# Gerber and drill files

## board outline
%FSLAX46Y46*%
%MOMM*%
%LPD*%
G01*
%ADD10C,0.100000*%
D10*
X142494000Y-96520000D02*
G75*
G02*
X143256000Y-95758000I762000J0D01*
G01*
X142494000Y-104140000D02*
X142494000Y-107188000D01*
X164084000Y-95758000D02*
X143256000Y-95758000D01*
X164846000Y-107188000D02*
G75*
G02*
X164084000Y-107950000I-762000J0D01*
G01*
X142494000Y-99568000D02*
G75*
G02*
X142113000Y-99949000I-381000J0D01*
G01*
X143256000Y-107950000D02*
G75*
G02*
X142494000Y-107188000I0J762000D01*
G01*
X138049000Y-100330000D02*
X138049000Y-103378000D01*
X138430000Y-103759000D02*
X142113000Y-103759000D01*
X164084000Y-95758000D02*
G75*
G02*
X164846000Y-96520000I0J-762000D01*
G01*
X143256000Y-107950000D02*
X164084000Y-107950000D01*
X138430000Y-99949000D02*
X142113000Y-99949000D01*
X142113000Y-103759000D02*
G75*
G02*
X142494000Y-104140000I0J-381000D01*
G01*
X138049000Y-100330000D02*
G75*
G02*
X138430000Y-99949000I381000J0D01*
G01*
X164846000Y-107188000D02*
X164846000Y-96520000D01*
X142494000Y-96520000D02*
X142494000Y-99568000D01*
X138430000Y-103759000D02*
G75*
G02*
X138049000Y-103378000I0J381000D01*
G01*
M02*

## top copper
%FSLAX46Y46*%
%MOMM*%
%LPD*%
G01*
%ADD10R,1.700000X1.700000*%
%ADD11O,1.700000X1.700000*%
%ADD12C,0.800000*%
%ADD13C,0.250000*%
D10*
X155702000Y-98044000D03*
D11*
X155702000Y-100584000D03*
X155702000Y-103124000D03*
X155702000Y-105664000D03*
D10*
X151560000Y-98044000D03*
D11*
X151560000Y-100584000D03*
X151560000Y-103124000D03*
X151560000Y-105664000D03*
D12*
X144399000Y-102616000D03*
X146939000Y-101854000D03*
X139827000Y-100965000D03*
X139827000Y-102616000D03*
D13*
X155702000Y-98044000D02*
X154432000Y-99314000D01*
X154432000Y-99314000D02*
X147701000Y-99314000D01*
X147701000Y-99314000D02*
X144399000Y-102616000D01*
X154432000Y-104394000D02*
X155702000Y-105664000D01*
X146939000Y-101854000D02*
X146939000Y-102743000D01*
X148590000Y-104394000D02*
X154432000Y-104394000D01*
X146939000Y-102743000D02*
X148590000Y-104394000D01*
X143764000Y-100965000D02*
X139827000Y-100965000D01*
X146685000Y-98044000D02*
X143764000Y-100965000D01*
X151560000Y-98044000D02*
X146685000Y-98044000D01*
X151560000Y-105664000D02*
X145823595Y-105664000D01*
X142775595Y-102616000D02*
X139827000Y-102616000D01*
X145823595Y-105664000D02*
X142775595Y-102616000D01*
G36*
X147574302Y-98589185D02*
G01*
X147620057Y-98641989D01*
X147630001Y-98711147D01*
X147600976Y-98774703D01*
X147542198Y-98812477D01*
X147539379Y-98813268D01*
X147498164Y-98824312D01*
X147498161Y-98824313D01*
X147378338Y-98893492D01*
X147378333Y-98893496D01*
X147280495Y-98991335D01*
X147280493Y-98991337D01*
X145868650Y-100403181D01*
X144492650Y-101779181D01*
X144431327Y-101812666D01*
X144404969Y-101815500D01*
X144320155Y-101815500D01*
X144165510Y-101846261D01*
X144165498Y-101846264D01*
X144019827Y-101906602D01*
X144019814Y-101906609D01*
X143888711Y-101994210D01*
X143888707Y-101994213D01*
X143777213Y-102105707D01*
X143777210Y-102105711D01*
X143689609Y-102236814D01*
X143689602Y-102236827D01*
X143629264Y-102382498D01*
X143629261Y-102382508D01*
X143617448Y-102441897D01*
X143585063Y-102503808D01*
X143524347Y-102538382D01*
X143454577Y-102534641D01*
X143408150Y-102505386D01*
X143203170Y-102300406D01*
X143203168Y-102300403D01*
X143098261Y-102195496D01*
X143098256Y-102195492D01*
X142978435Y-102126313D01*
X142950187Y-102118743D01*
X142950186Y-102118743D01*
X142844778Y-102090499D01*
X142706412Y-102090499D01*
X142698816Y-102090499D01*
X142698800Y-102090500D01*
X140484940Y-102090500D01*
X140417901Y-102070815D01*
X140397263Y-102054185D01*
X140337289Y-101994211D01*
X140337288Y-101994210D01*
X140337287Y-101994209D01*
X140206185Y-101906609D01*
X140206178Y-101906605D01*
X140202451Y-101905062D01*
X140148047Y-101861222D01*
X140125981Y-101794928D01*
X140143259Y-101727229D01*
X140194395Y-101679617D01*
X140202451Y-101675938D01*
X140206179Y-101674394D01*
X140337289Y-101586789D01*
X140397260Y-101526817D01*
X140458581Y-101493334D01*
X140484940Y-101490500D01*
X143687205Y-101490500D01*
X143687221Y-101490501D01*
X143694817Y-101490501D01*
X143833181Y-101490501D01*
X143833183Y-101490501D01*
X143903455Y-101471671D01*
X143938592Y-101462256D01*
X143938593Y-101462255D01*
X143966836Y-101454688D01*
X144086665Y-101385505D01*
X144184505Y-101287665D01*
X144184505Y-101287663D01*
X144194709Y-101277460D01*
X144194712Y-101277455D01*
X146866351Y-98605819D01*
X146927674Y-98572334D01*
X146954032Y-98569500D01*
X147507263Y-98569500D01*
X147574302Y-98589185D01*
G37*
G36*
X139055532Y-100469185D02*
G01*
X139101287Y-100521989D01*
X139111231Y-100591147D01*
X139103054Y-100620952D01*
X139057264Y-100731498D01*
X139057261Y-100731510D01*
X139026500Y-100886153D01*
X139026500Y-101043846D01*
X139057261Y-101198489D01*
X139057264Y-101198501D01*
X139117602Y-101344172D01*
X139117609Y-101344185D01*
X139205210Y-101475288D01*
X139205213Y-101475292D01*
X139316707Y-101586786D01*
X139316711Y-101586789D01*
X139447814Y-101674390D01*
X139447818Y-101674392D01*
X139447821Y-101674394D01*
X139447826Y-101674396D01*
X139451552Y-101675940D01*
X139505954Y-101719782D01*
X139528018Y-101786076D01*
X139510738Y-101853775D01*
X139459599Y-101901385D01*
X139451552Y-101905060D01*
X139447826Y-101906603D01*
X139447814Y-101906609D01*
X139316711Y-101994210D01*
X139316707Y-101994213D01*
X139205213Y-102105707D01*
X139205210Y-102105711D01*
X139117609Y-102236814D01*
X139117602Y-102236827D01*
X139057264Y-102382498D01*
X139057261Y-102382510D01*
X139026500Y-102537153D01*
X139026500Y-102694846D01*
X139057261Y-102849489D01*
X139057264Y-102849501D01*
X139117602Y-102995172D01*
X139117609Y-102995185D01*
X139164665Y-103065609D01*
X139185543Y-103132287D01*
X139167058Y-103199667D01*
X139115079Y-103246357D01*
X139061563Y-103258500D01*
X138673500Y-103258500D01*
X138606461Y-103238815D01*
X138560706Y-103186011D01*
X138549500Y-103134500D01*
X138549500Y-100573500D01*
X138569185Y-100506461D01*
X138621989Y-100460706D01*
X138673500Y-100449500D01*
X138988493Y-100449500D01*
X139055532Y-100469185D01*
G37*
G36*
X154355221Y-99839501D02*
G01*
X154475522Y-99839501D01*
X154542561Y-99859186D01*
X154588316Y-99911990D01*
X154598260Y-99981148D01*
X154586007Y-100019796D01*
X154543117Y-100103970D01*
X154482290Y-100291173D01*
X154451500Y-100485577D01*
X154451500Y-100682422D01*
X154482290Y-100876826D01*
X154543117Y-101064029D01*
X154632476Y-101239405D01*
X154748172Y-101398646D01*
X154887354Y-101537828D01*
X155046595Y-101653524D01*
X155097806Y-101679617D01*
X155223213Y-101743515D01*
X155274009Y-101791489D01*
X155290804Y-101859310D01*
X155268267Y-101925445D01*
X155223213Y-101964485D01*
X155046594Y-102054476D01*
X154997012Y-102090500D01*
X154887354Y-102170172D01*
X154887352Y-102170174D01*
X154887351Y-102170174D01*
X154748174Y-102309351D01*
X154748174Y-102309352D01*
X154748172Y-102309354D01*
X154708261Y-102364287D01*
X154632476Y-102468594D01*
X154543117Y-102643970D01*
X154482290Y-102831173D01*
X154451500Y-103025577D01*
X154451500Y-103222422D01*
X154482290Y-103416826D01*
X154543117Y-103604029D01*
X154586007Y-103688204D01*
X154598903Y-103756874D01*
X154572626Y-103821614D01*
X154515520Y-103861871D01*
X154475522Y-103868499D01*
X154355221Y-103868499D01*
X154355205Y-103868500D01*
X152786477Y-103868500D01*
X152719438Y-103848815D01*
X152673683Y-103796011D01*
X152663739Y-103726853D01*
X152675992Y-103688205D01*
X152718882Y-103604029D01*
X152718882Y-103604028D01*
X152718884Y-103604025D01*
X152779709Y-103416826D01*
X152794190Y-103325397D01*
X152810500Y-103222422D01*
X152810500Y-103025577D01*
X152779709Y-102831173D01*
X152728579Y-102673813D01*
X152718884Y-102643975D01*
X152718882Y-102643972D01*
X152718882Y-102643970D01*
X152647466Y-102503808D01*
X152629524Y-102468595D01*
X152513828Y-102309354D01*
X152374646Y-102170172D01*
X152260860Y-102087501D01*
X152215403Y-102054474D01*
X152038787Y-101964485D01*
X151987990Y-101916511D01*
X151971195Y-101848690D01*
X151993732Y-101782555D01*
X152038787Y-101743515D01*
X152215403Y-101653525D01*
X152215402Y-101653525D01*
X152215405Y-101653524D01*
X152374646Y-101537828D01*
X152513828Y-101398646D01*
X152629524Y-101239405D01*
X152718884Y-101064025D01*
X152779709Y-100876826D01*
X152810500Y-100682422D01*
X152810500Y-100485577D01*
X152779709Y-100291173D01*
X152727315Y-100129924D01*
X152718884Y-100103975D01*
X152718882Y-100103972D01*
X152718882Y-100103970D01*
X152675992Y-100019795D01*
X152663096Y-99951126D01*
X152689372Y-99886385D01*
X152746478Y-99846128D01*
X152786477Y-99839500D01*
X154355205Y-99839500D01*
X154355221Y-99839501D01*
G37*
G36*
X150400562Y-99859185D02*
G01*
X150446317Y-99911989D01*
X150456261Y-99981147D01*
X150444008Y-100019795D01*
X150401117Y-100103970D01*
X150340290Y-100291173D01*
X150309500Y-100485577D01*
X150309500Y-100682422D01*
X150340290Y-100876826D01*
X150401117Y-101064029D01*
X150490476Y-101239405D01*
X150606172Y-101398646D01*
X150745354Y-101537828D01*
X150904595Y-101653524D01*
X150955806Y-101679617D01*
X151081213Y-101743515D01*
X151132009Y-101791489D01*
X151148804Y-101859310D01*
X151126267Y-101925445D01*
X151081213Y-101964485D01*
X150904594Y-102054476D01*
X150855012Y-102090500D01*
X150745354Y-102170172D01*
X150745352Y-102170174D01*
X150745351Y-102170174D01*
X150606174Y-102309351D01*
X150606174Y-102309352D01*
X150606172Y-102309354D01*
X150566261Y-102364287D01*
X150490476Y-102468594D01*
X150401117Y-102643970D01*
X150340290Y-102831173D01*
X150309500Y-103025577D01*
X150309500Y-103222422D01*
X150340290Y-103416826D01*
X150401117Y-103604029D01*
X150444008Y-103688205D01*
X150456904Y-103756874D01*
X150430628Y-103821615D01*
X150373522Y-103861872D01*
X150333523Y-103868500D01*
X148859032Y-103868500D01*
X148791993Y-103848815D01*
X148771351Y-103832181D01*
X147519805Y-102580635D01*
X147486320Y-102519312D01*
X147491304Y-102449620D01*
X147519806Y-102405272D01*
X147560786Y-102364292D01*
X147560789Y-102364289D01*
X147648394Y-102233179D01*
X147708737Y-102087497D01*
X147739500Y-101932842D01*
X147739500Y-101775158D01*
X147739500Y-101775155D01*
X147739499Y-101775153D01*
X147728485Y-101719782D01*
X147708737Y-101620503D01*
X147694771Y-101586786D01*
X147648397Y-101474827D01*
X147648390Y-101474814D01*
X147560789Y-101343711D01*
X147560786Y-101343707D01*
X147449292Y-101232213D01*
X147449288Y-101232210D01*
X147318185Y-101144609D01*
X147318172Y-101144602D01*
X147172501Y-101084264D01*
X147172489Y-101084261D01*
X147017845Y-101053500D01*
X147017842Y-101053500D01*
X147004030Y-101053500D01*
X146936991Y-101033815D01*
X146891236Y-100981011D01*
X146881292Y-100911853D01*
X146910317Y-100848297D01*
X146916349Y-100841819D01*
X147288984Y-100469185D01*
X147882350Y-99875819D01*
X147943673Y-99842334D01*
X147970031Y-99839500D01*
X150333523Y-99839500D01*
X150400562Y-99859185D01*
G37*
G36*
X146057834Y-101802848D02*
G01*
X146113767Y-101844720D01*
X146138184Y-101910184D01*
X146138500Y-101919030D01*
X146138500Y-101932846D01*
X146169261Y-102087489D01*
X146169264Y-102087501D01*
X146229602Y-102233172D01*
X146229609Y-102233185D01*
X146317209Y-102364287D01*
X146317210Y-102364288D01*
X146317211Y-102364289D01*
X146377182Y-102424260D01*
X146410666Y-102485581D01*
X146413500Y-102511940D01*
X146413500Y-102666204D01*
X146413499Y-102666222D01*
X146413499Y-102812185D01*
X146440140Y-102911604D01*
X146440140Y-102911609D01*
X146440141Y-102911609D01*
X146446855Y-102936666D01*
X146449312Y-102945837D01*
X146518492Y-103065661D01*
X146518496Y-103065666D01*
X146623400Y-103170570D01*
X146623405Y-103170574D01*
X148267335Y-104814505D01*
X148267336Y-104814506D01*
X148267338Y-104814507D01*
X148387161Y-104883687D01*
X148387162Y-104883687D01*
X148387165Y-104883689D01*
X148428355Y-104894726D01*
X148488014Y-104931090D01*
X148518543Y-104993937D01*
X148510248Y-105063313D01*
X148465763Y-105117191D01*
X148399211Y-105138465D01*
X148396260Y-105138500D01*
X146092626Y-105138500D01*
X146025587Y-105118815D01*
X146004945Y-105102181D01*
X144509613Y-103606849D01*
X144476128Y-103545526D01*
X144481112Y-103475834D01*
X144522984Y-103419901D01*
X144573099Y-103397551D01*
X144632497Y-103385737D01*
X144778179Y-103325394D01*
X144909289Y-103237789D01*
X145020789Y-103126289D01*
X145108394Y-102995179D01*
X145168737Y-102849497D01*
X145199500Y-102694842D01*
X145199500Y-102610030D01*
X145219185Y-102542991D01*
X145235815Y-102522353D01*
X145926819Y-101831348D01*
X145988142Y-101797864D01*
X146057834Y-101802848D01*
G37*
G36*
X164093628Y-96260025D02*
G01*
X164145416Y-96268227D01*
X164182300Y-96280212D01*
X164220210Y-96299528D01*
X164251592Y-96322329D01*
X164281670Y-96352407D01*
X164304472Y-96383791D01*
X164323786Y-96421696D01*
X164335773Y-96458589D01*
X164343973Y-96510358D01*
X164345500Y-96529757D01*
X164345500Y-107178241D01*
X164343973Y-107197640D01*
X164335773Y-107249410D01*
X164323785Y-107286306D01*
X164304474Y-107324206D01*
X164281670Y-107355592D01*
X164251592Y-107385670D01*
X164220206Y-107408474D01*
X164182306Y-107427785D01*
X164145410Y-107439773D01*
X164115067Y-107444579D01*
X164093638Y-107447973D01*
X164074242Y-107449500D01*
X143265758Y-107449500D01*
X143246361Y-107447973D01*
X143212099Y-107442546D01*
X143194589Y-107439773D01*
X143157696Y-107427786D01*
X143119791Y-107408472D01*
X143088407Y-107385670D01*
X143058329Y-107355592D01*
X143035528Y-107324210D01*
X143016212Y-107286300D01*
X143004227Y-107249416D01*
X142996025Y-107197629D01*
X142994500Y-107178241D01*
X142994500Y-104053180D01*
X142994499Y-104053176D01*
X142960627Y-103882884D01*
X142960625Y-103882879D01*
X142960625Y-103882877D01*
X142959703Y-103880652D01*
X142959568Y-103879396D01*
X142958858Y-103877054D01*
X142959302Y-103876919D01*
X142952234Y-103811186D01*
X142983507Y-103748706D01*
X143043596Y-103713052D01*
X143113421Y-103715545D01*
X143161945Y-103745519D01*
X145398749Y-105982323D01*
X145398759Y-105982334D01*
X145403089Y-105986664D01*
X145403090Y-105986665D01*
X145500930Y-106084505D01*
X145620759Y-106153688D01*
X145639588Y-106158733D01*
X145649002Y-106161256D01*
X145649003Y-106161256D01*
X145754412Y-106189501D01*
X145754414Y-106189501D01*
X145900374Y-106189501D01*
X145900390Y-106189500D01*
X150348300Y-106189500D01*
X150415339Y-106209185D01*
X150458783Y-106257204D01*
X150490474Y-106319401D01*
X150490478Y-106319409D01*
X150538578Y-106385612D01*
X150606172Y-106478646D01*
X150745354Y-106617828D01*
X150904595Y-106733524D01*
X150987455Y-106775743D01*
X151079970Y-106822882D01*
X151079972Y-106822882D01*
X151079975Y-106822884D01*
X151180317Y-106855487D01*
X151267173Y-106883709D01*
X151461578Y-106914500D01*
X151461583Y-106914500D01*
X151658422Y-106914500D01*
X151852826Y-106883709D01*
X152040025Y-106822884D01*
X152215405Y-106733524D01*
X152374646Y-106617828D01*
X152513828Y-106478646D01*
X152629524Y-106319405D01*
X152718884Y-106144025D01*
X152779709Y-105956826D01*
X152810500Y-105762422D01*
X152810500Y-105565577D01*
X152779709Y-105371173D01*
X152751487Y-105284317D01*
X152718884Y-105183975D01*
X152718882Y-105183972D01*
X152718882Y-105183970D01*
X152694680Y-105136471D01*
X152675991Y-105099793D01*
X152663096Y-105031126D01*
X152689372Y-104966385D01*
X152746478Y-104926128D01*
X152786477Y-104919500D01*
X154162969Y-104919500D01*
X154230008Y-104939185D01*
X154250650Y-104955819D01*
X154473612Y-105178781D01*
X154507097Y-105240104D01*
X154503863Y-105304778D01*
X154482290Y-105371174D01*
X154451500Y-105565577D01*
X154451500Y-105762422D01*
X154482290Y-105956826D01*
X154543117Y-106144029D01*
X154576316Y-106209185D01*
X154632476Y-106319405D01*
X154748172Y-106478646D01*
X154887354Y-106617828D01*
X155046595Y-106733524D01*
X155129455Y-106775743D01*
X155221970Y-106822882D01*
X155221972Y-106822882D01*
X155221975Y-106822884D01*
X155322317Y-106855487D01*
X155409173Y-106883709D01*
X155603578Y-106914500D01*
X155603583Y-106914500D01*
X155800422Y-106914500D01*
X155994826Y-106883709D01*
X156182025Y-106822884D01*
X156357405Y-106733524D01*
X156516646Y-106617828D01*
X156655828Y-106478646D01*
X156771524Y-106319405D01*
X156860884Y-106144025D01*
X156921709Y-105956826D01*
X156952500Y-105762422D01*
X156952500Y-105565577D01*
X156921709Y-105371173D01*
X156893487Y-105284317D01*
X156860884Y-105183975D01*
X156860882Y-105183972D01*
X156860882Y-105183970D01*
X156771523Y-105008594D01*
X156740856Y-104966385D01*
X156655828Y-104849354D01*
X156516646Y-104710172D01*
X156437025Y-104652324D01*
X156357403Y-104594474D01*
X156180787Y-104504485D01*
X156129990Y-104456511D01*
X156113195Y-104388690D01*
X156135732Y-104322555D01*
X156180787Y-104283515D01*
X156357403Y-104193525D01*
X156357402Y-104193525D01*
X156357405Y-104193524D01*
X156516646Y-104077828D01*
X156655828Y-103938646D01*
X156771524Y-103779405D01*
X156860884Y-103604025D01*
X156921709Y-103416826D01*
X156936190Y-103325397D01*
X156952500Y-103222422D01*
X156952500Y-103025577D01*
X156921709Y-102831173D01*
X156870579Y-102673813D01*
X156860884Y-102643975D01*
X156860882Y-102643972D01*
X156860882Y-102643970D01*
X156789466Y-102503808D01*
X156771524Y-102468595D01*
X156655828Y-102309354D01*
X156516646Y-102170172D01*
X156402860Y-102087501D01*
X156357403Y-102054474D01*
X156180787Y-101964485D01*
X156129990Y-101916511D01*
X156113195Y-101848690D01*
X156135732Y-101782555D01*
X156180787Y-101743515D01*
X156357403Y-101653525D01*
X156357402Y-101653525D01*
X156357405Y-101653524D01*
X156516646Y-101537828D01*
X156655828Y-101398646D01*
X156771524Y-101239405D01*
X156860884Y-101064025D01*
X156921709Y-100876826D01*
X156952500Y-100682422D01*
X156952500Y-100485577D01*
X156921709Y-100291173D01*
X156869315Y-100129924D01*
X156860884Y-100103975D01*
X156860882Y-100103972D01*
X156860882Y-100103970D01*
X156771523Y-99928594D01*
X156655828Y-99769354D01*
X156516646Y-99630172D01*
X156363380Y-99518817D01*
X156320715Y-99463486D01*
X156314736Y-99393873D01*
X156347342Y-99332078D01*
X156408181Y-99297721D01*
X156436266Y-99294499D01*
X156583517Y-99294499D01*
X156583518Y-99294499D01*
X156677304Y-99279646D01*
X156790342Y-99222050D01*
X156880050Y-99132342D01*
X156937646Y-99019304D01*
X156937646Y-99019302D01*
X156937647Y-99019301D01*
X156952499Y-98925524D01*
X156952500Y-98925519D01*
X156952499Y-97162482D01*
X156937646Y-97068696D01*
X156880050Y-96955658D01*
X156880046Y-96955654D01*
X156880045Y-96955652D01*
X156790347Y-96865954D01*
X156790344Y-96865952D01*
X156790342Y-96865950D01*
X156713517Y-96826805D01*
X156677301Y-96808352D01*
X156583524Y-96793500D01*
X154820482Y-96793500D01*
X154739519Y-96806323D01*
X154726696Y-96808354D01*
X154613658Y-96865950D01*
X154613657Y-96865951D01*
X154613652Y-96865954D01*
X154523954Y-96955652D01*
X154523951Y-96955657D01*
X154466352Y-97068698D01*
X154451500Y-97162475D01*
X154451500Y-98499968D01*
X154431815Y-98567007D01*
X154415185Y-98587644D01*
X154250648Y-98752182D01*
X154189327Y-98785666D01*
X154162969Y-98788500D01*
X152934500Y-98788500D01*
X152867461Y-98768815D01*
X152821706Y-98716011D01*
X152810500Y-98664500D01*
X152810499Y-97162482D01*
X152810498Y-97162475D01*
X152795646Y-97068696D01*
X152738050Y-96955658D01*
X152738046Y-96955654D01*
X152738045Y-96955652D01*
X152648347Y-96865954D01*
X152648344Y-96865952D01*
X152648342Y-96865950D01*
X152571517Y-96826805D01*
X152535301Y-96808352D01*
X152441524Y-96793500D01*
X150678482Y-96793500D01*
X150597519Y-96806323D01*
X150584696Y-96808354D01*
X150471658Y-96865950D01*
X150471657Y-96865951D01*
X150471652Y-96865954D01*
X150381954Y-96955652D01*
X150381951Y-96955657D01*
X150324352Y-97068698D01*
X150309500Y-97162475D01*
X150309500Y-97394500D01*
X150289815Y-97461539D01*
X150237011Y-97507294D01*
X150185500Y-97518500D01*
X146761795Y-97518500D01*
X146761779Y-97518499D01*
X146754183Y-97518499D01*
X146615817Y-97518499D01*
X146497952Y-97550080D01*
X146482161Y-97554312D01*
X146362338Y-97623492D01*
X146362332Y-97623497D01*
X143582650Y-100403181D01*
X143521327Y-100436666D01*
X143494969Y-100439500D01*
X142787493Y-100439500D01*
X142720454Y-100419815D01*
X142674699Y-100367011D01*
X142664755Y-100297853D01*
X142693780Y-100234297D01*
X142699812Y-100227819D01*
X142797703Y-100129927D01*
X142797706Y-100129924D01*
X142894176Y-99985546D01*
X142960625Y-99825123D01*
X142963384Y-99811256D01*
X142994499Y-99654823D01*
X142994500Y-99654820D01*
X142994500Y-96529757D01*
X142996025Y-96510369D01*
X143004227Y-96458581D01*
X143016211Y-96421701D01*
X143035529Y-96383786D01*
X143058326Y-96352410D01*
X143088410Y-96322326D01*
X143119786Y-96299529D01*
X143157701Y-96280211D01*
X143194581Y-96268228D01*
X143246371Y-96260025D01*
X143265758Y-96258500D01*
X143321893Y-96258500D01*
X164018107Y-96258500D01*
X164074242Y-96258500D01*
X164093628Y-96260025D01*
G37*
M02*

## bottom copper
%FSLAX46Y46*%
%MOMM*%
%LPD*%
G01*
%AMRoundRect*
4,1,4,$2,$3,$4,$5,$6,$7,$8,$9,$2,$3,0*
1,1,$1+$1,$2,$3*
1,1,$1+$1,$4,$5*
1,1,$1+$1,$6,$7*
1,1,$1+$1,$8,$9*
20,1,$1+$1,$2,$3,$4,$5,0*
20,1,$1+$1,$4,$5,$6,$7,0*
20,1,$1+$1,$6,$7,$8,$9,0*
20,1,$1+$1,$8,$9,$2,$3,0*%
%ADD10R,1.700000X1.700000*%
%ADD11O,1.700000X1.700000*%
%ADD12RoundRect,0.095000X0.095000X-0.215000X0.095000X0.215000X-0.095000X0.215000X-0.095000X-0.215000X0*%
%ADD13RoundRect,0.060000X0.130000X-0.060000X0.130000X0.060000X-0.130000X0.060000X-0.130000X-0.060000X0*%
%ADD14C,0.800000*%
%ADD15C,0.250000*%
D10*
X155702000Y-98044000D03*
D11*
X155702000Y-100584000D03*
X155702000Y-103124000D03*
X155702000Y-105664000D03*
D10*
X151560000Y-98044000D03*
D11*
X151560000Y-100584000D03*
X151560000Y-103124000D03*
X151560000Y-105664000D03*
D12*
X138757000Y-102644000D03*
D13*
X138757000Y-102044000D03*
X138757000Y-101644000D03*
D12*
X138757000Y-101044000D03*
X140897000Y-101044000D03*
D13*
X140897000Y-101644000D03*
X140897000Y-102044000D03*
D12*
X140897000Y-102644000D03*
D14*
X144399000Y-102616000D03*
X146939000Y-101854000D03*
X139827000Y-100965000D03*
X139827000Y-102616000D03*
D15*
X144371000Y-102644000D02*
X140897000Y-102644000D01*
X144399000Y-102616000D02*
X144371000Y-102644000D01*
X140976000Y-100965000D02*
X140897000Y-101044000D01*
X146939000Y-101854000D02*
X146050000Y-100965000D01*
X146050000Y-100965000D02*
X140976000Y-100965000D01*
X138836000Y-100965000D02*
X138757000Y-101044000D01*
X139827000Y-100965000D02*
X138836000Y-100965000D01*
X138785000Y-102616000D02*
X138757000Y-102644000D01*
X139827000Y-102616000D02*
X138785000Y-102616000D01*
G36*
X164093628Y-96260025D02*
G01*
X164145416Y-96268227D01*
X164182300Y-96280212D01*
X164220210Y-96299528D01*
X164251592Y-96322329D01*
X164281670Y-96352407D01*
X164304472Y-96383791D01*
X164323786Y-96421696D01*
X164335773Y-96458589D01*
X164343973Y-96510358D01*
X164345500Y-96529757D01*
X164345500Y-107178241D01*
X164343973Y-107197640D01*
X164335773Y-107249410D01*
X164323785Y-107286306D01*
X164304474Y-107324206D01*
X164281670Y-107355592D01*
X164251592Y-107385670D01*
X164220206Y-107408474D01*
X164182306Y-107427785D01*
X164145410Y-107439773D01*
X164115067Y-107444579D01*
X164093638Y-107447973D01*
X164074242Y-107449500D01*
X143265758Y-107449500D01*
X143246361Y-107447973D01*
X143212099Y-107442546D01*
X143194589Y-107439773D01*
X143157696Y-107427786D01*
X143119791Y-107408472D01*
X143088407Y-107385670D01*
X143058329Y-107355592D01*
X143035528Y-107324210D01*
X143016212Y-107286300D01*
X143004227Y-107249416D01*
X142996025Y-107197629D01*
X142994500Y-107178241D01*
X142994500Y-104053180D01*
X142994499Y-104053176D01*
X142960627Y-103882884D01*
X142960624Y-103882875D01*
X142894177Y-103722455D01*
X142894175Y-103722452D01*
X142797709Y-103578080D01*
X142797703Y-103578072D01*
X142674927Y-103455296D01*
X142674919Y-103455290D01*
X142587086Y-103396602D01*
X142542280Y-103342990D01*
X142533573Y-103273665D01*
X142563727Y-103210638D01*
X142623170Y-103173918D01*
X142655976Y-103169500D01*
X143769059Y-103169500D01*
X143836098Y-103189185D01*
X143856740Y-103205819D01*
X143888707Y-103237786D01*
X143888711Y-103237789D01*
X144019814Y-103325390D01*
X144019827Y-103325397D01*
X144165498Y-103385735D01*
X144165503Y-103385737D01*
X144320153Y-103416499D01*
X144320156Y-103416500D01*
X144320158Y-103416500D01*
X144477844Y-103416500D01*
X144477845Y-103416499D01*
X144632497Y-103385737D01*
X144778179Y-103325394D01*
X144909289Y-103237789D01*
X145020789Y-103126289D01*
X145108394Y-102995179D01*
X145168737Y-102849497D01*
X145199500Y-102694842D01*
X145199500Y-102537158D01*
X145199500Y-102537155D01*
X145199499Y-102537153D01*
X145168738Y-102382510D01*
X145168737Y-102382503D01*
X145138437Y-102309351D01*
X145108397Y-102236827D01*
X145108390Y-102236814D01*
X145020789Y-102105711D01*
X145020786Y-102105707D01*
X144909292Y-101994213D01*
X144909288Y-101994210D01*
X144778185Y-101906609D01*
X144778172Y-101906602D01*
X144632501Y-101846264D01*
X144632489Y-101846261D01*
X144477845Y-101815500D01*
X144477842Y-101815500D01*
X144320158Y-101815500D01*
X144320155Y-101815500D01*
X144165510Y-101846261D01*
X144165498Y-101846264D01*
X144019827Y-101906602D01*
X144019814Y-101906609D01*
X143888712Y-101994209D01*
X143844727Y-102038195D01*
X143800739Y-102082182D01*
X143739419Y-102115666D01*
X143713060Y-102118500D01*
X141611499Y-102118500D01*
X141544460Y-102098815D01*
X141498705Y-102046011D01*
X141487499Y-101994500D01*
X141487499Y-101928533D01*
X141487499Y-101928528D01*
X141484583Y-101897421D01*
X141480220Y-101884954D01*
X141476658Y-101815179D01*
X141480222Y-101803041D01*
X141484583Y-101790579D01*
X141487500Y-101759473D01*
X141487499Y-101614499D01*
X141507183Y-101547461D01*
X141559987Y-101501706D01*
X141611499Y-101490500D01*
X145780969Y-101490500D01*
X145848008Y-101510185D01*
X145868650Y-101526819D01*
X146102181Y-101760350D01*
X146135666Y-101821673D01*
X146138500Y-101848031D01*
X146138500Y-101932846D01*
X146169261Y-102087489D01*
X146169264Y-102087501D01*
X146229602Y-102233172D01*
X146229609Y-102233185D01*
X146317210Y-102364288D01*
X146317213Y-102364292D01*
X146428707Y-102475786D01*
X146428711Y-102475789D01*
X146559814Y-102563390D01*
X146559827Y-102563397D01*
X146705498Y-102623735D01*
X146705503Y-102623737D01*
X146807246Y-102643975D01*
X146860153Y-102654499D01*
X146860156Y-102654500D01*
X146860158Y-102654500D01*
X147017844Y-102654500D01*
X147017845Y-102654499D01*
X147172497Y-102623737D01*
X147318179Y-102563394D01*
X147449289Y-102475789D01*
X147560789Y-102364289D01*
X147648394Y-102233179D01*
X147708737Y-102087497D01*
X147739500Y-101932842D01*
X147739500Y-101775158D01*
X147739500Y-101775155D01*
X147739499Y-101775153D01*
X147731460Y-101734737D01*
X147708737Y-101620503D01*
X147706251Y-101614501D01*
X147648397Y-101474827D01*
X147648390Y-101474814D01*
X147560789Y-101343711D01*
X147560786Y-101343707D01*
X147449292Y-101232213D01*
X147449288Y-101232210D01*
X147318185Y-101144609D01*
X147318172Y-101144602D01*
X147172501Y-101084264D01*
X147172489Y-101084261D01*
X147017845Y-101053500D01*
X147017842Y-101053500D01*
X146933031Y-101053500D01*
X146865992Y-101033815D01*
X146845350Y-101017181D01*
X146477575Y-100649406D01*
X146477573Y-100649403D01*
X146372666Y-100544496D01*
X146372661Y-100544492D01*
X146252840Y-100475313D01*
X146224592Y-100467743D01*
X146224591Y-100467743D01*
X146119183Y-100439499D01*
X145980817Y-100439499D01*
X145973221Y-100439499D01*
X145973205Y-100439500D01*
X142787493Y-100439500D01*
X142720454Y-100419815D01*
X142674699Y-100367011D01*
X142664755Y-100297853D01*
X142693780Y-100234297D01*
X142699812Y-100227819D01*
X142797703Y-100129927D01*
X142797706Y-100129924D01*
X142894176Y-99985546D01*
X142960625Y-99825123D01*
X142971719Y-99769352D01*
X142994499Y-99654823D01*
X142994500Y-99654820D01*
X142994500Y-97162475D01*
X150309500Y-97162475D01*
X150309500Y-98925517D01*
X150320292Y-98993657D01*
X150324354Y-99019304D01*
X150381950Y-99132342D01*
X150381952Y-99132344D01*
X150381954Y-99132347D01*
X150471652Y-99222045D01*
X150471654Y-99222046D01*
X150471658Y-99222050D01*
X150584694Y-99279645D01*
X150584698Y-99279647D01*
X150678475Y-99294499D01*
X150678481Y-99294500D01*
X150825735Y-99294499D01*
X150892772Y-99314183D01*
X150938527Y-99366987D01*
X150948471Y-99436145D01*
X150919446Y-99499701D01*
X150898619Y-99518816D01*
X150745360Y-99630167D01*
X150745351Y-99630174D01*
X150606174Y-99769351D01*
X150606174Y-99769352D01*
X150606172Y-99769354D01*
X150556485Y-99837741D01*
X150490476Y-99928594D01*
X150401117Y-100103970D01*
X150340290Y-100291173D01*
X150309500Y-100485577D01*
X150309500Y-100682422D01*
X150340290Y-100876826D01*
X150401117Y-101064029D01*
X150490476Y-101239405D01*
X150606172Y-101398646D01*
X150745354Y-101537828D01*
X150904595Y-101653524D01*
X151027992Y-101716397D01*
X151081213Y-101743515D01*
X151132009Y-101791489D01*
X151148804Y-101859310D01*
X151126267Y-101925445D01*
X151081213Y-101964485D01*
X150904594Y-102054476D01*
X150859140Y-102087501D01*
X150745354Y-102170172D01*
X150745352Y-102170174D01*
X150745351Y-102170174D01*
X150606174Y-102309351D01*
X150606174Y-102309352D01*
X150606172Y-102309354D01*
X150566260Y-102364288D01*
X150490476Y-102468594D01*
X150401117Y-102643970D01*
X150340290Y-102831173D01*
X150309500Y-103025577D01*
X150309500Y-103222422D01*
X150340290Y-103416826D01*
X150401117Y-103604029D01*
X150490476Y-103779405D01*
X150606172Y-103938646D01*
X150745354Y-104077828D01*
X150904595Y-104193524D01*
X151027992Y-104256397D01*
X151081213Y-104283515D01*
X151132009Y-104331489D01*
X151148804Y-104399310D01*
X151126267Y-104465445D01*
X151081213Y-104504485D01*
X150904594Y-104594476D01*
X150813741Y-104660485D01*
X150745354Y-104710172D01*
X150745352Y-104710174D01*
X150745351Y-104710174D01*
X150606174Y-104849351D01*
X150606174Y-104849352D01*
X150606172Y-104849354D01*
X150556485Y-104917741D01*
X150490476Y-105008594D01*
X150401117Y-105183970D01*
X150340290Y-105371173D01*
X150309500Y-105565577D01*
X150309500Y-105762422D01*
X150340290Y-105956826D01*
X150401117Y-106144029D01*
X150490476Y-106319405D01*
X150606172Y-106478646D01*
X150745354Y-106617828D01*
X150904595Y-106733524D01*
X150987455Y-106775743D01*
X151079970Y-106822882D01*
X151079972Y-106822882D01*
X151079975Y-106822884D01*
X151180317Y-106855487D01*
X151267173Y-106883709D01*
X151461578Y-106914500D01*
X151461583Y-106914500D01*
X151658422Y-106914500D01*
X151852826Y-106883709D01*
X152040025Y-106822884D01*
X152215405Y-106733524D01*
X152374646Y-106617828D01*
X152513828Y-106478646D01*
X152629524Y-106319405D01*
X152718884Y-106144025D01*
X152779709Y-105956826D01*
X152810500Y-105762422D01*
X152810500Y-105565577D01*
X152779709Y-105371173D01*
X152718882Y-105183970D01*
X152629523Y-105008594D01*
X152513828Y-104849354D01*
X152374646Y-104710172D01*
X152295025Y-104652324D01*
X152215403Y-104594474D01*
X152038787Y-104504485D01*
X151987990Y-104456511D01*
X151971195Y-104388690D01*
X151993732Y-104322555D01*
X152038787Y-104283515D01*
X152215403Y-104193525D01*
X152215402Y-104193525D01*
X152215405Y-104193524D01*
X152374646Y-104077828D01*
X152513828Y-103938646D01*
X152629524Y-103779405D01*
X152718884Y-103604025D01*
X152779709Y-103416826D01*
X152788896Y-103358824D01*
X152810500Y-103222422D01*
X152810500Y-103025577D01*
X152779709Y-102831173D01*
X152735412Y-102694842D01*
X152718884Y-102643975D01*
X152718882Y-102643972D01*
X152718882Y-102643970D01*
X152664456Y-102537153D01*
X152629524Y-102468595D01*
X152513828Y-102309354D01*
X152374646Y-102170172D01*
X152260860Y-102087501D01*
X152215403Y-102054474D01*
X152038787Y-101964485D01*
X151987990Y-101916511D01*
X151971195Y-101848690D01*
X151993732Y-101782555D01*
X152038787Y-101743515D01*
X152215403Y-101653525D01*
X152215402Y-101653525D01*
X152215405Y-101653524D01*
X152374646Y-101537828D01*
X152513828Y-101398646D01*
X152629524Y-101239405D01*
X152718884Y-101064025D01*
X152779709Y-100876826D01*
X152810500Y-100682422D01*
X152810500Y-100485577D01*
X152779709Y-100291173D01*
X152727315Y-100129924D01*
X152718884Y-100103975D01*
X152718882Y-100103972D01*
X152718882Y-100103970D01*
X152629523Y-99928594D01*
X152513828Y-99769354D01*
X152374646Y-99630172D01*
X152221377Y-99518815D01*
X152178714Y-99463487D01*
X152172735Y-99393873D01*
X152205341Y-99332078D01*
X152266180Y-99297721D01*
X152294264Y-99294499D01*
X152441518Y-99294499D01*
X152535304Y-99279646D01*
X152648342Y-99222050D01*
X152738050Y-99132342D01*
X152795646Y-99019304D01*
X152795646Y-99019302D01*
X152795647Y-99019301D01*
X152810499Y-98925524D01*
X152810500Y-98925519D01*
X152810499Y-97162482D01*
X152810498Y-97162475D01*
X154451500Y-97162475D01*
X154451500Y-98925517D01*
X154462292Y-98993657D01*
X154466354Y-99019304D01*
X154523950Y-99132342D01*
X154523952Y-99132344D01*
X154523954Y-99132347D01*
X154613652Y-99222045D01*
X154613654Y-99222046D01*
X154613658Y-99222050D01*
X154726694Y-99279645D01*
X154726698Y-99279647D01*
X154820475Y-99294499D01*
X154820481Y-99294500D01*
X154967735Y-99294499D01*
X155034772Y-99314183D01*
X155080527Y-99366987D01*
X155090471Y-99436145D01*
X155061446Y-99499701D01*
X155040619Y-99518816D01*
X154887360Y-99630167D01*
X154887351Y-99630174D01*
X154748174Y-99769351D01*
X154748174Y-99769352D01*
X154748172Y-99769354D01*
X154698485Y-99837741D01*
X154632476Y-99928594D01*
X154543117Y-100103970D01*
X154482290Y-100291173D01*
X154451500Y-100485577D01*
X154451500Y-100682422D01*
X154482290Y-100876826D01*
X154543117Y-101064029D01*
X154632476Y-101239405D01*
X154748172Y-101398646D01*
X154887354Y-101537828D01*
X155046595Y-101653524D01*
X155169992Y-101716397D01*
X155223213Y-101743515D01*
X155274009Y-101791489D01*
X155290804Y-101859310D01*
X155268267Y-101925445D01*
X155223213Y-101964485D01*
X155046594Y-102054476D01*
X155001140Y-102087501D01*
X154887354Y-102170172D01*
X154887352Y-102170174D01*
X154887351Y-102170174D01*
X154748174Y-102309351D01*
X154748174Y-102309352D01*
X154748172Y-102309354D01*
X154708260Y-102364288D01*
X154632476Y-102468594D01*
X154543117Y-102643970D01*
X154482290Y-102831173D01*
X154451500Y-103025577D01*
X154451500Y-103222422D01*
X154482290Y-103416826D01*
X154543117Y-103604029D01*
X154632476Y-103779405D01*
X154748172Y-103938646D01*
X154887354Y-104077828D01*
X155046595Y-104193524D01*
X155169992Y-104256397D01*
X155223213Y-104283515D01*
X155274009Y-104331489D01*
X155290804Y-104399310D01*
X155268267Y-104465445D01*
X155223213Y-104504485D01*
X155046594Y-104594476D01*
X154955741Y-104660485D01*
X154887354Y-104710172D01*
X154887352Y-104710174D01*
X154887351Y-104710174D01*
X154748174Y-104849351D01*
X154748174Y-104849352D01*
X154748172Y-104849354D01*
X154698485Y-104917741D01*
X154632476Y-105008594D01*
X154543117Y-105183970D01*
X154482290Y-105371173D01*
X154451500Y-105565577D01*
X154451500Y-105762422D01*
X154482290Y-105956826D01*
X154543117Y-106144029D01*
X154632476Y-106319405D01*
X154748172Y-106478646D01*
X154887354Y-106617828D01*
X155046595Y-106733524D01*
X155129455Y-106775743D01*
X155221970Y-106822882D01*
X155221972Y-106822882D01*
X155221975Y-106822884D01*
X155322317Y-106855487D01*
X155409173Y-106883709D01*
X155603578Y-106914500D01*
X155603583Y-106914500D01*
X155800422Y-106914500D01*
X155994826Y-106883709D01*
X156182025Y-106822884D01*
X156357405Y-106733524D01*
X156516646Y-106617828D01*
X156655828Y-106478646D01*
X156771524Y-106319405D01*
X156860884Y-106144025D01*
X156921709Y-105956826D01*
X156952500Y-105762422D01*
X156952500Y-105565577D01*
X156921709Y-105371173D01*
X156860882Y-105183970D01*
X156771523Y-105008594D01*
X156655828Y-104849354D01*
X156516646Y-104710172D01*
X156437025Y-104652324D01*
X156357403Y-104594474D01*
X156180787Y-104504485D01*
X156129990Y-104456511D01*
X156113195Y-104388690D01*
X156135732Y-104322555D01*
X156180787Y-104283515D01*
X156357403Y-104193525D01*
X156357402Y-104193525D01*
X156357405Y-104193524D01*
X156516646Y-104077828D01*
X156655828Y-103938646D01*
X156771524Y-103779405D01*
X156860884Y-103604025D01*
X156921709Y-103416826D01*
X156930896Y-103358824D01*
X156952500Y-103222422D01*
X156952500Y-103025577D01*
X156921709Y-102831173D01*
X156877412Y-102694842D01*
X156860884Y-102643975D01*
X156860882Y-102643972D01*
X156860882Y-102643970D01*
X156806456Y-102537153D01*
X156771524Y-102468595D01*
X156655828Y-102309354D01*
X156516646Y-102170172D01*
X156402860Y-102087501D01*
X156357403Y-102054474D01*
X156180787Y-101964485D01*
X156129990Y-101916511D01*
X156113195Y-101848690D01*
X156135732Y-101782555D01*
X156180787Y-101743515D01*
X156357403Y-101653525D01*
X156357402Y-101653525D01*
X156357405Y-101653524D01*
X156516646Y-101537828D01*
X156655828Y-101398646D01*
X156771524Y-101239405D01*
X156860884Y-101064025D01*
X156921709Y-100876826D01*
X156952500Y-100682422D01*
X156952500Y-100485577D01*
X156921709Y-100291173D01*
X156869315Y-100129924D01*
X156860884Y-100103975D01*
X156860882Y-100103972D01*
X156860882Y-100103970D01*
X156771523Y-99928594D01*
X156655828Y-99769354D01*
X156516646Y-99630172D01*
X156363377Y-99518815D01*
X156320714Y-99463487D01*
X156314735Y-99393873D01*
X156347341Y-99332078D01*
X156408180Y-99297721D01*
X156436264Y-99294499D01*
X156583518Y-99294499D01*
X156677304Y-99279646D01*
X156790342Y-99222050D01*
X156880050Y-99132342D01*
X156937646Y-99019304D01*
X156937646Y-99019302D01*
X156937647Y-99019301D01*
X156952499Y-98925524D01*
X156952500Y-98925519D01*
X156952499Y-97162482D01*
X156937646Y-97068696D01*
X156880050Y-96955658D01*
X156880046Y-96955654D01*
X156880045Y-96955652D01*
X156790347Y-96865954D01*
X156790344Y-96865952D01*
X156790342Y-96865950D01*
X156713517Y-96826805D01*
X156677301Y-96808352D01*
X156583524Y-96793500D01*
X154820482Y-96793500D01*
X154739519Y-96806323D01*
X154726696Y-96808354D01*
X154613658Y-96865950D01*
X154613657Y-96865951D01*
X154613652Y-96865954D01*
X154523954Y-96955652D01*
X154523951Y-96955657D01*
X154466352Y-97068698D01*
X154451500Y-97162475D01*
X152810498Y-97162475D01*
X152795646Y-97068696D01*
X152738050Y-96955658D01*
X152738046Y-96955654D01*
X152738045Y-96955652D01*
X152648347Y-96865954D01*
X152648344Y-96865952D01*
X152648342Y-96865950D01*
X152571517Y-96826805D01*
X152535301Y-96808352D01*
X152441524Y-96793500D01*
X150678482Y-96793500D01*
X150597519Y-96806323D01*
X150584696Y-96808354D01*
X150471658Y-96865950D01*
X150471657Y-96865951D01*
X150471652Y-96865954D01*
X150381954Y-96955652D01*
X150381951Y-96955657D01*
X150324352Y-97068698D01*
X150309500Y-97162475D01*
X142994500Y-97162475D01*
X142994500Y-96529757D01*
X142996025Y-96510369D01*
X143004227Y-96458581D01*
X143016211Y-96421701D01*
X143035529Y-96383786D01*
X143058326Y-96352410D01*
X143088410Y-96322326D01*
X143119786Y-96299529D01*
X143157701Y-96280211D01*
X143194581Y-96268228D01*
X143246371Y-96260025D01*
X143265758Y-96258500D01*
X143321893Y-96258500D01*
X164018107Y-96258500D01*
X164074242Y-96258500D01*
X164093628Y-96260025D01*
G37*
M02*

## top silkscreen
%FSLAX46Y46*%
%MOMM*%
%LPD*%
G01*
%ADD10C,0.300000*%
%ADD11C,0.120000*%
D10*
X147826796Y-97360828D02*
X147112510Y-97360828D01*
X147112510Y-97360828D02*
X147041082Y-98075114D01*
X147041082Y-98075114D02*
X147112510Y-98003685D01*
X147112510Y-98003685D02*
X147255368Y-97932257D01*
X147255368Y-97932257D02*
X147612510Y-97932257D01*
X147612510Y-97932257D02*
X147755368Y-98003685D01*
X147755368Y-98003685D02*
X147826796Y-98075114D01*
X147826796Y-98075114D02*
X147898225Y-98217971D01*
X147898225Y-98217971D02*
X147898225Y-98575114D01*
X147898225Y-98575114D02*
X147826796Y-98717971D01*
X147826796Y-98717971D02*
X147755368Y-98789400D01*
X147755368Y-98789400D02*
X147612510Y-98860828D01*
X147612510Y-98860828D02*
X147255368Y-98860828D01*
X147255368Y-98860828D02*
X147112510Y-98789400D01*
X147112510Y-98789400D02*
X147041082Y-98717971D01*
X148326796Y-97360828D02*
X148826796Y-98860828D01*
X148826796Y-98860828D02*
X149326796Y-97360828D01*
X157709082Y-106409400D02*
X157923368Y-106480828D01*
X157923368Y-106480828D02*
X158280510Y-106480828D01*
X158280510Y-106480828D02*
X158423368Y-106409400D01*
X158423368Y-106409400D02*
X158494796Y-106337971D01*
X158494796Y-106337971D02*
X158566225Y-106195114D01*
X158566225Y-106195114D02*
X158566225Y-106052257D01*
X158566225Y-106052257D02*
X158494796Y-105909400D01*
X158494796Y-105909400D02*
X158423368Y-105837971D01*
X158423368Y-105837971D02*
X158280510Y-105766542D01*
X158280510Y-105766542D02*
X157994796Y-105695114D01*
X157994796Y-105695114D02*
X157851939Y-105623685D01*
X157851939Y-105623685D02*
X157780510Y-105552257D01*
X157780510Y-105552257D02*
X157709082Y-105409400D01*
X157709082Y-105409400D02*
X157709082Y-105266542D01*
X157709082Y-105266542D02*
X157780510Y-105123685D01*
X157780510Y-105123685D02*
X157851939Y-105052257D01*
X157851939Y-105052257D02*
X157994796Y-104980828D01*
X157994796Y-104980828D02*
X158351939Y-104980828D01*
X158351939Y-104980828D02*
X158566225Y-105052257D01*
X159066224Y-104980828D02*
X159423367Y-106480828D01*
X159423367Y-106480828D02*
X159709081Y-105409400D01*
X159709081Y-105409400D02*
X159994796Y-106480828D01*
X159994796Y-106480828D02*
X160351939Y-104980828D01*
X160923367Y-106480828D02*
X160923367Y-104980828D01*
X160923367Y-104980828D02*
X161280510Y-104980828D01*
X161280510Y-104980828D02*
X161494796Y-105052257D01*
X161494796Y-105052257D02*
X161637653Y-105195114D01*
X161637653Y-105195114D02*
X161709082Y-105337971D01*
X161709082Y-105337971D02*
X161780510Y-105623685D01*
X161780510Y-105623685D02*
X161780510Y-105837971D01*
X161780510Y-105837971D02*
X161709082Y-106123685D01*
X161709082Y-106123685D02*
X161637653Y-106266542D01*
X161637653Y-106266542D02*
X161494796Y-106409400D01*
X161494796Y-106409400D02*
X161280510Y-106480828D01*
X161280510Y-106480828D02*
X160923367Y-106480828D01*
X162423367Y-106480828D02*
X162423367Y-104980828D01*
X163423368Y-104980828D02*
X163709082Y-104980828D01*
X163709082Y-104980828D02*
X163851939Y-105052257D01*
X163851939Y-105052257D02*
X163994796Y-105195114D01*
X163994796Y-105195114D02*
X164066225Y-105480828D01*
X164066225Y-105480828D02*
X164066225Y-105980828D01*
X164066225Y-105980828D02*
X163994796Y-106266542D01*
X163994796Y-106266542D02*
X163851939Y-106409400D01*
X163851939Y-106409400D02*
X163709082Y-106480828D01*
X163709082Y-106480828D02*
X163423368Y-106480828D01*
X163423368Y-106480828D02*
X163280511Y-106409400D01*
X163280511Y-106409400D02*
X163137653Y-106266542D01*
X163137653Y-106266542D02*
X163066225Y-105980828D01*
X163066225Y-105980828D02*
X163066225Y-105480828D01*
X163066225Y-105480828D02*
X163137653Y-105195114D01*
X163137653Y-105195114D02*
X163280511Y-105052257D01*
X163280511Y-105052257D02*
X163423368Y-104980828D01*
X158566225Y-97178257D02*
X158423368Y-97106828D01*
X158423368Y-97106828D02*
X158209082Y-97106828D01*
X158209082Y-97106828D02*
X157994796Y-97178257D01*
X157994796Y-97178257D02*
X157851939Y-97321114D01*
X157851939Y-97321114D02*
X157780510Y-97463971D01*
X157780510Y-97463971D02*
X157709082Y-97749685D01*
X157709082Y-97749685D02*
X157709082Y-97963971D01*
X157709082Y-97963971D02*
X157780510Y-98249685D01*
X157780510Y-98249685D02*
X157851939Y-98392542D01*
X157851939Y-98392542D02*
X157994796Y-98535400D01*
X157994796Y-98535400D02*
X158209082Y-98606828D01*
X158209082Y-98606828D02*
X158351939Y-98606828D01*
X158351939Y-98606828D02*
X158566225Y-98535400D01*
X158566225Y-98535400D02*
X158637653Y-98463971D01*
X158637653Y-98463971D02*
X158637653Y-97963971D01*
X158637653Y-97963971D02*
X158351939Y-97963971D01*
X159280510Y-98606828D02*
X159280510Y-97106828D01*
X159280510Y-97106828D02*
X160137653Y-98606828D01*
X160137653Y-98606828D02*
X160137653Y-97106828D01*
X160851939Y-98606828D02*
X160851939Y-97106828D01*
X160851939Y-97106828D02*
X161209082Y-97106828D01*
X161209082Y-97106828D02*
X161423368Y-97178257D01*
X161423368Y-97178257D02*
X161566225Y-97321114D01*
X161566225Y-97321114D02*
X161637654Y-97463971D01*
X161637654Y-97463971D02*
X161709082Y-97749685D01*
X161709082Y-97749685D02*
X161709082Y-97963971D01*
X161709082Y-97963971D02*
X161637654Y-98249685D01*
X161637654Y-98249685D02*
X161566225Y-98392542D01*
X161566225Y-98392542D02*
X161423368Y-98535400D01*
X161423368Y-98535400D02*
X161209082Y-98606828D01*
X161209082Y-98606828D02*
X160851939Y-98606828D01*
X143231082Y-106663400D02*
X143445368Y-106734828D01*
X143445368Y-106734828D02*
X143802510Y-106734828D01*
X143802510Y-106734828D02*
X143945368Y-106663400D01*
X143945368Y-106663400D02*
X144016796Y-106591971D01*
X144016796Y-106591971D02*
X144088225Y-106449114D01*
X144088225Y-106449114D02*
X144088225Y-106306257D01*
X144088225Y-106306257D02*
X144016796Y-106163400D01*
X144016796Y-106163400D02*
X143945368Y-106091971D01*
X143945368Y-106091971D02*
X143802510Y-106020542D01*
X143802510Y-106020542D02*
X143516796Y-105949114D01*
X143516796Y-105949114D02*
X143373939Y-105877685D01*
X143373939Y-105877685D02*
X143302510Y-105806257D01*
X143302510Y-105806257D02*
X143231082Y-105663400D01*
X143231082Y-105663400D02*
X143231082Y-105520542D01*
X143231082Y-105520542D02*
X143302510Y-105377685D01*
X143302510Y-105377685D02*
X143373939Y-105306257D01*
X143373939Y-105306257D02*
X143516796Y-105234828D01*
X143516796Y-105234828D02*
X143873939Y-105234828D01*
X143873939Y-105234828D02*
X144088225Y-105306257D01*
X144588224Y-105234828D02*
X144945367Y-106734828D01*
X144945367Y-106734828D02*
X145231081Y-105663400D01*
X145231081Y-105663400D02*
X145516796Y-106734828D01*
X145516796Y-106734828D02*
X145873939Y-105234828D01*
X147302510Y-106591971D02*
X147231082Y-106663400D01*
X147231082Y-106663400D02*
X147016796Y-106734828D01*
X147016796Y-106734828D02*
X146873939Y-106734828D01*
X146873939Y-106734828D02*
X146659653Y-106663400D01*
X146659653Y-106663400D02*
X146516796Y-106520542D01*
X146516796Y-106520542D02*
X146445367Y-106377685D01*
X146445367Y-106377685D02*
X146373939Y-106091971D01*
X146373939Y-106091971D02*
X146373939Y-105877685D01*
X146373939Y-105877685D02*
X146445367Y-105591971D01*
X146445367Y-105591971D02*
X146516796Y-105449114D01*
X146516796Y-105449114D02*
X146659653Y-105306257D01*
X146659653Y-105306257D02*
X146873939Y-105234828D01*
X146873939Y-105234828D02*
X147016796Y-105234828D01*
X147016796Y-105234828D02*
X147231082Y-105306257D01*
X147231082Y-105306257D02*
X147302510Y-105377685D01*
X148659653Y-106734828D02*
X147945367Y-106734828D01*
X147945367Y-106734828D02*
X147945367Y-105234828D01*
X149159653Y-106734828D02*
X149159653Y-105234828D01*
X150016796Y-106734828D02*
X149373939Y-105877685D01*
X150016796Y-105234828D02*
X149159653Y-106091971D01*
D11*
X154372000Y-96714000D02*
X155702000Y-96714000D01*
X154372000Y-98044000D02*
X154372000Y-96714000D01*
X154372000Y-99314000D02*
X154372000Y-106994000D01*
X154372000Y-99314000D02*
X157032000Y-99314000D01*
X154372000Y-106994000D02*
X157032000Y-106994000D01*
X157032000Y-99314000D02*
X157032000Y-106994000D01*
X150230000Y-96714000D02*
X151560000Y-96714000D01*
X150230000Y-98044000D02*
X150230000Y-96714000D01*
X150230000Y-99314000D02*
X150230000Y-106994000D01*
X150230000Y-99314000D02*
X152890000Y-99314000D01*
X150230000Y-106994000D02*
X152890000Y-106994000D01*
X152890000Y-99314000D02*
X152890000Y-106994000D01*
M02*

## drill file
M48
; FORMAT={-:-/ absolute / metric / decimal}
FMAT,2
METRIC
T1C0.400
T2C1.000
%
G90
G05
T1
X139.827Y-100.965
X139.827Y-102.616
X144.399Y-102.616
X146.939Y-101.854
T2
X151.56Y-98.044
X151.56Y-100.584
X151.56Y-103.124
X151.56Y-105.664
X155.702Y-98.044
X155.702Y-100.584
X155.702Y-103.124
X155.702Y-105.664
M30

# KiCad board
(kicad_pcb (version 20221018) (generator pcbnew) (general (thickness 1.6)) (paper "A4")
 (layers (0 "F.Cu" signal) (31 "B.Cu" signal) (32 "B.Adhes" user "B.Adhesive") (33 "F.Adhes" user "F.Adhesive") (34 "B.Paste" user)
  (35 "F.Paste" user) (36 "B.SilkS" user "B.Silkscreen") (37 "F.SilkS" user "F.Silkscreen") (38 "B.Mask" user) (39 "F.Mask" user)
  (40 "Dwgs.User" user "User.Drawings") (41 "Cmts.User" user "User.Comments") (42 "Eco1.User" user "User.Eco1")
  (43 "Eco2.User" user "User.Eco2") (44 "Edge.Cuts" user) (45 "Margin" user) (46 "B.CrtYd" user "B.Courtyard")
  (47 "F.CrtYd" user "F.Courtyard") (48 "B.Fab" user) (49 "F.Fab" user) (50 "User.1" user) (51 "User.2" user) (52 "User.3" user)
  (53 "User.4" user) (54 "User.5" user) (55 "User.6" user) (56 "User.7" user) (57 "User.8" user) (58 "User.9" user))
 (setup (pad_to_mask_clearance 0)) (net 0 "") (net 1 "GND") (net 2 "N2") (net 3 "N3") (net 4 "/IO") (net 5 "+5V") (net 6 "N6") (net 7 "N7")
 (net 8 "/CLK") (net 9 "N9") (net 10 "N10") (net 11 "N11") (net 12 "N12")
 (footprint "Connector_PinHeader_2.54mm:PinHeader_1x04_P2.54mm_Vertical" (layer "F.Cu") (at 155.702 98.044)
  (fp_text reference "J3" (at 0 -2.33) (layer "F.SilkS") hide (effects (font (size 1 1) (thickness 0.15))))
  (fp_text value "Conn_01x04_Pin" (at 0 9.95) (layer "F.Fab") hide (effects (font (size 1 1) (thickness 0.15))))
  (fp_line (start -1.33 -1.33) (end 0 -1.33) (stroke (width 0.12) (type solid)) (layer "F.SilkS"))
  (fp_line (start -1.33 0) (end -1.33 -1.33) (stroke (width 0.12) (type solid)) (layer "F.SilkS"))
  (fp_line (start -1.33 1.27) (end -1.33 8.95) (stroke (width 0.12) (type solid)) (layer "F.SilkS"))
  (fp_line (start -1.33 1.27) (end 1.33 1.27) (stroke (width 0.12) (type solid)) (layer "F.SilkS"))
  (fp_line (start -1.33 8.95) (end 1.33 8.95) (stroke (width 0.12) (type solid)) (layer "F.SilkS"))
  (fp_line (start 1.33 1.27) (end 1.33 8.95) (stroke (width 0.12) (type solid)) (layer "F.SilkS"))
  (pad "1" thru_hole rect (at 0 0) (size 1.7 1.7) (drill 1) (layers "*.Cu" "*.Mask") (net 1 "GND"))
  (pad "2" thru_hole oval (at 0 2.54) (size 1.7 1.7) (drill 1) (layers "*.Cu" "*.Mask") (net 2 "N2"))
  (pad "3" thru_hole oval (at 0 5.08) (size 1.7 1.7) (drill 1) (layers "*.Cu" "*.Mask") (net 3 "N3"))
  (pad "4" thru_hole oval (at 0 7.62) (size 1.7 1.7) (drill 1) (layers "*.Cu" "*.Mask") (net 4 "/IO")))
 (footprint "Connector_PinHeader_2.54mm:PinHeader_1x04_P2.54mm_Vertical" (layer "F.Cu") (at 151.56 98.044)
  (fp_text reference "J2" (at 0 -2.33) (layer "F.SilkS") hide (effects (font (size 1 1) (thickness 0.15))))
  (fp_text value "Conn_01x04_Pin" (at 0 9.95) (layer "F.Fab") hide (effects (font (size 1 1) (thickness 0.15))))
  (fp_line (start -1.33 -1.33) (end 0 -1.33) (stroke (width 0.12) (type solid)) (layer "F.SilkS"))
  (fp_line (start -1.33 0) (end -1.33 -1.33) (stroke (width 0.12) (type solid)) (layer "F.SilkS"))
  (fp_line (start -1.33 1.27) (end -1.33 8.95) (stroke (width 0.12) (type solid)) (layer "F.SilkS"))
  (fp_line (start -1.33 1.27) (end 1.33 1.27) (stroke (width 0.12) (type solid)) (layer "F.SilkS"))
  (fp_line (start -1.33 8.95) (end 1.33 8.95) (stroke (width 0.12) (type solid)) (layer "F.SilkS"))
  (fp_line (start 1.33 1.27) (end 1.33 8.95) (stroke (width 0.12) (type solid)) (layer "F.SilkS"))
  (pad "1" thru_hole rect (at 0 0) (size 1.7 1.7) (drill 1) (layers "*.Cu" "*.Mask") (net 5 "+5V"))
  (pad "2" thru_hole oval (at 0 2.54) (size 1.7 1.7) (drill 1) (layers "*.Cu" "*.Mask") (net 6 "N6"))
  (pad "3" thru_hole oval (at 0 5.08) (size 1.7 1.7) (drill 1) (layers "*.Cu" "*.Mask") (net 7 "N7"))
  (pad "4" thru_hole oval (at 0 7.62) (size 1.7 1.7) (drill 1) (layers "*.Cu" "*.Mask") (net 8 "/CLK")))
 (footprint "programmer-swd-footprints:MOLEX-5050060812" (layer "B.Cu") (at 139.827 101.844 90)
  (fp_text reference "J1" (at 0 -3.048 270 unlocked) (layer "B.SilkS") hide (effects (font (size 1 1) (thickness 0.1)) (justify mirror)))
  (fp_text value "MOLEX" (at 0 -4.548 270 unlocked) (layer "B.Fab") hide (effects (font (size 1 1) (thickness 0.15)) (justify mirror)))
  (pad "1" smd roundrect (at -0.8 -1.07 90) (size 0.62 0.38) (layers "B.Cu" "B.Paste" "B.Mask") (roundrect_rratio 0.25) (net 8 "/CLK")
   (thermal_bridge_angle 45))
  (pad "2" smd roundrect (at -0.2 -1.07 90) (size 0.24 0.38) (layers "B.Cu" "B.Paste" "B.Mask") (roundrect_rratio 0.25) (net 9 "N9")
   (thermal_bridge_angle 45))
  (pad "3" smd roundrect (at 0.2 -1.07 90) (size 0.24 0.38) (layers "B.Cu" "B.Paste" "B.Mask") (roundrect_rratio 0.25) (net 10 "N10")
   (thermal_bridge_angle 45))
  (pad "4" smd roundrect (at 0.8 -1.07 90) (size 0.62 0.38) (layers "B.Cu" "B.Paste" "B.Mask") (roundrect_rratio 0.25) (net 5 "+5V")
   (thermal_bridge_angle 45))
  (pad "5" smd roundrect (at 0.8 1.07 90) (size 0.62 0.38) (layers "B.Cu" "B.Paste" "B.Mask") (roundrect_rratio 0.25) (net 4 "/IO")
   (thermal_bridge_angle 45))
  (pad "6" smd roundrect (at 0.2 1.07 90) (size 0.24 0.38) (layers "B.Cu" "B.Paste" "B.Mask") (roundrect_rratio 0.25) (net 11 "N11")
   (thermal_bridge_angle 45))
  (pad "7" smd roundrect (at -0.2 1.07 90) (size 0.24 0.38) (layers "B.Cu" "B.Paste" "B.Mask") (roundrect_rratio 0.25) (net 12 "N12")
   (thermal_bridge_angle 45))
  (pad "8" smd roundrect (at -0.8 1.07 90) (size 0.62 0.38) (layers "B.Cu" "B.Paste" "B.Mask") (roundrect_rratio 0.25) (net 1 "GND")
   (thermal_bridge_angle 45)))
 (gr_arc (start 142.494 96.52) (mid 142.717185 95.981185) (end 143.256 95.758) (stroke (width 0.1) (type default)) (layer "Edge.Cuts"))
 (gr_line (start 142.494 104.14) (end 142.494 107.188) (stroke (width 0.1) (type default)) (layer "Edge.Cuts"))
 (gr_line (start 164.084 95.758) (end 143.256 95.758) (stroke (width 0.1) (type default)) (layer "Edge.Cuts"))
 (gr_arc (start 164.846 107.188) (mid 164.622815 107.726815) (end 164.084 107.95) (stroke (width 0.1) (type default)) (layer "Edge.Cuts"))
 (gr_arc (start 142.494 99.568) (mid 142.382408 99.837408) (end 142.113 99.949) (stroke (width 0.1) (type default)) (layer "Edge.Cuts"))
 (gr_arc (start 143.256 107.95) (mid 142.717185 107.726815) (end 142.494 107.188) (stroke (width 0.1) (type default)) (layer "Edge.Cuts"))
 (gr_line (start 138.049 100.33) (end 138.049 103.378) (stroke (width 0.1) (type default)) (layer "Edge.Cuts"))
 (gr_line (start 138.43 103.759) (end 142.113 103.759) (stroke (width 0.1) (type default)) (layer "Edge.Cuts"))
 (gr_arc (start 164.084 95.758) (mid 164.622815 95.981185) (end 164.846 96.52) (stroke (width 0.1) (type default)) (layer "Edge.Cuts"))
 (gr_line (start 143.256 107.95) (end 164.084 107.95) (stroke (width 0.1) (type default)) (layer "Edge.Cuts"))
 (gr_line (start 138.43 99.949) (end 142.113 99.949) (stroke (width 0.1) (type default)) (layer "Edge.Cuts"))
 (gr_arc (start 142.113 103.759) (mid 142.382408 103.870592) (end 142.494 104.14) (stroke (width 0.1) (type default)) (layer "Edge.Cuts"))
 (gr_arc (start 138.049 100.33) (mid 138.160592 100.060592) (end 138.43 99.949) (stroke (width 0.1) (type default)) (layer "Edge.Cuts"))
 (gr_line (start 164.846 107.188) (end 164.846 96.52) (stroke (width 0.1) (type default)) (layer "Edge.Cuts"))
 (gr_line (start 142.494 96.52) (end 142.494 99.568) (stroke (width 0.1) (type default)) (layer "Edge.Cuts"))
 (gr_arc (start 138.43 103.759) (mid 138.160592 103.647408) (end 138.049 103.378) (stroke (width 0.1) (type default)) (layer "Edge.Cuts"))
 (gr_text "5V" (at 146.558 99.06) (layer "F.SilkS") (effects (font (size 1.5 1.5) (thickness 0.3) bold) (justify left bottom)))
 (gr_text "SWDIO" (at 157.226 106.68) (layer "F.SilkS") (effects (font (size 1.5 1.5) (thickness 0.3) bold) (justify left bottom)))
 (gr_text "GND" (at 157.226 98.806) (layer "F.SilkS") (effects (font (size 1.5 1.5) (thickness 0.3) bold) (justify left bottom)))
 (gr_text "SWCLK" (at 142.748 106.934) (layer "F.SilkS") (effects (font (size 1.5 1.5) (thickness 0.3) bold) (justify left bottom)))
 (segment (start 155.702 98.044) (end 154.432 99.314) (width 0.25) (layer "F.Cu") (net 1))
 (segment (start 154.432 99.314) (end 147.701 99.314) (width 0.25) (layer "F.Cu") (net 1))
 (segment (start 147.701 99.314) (end 144.399 102.616) (width 0.25) (layer "F.Cu") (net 1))
 (via (at 144.399 102.616) (size 0.8) (drill 0.4) (layers "F.Cu" "B.Cu") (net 1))
 (segment (start 144.371 102.644) (end 140.897 102.644) (width 0.25) (layer "B.Cu") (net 1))
 (segment (start 144.399 102.616) (end 144.371 102.644) (width 0.25) (layer "B.Cu") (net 1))
 (segment (start 154.432 104.394) (end 155.702 105.664) (width 0.25) (layer "F.Cu") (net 4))
 (segment (start 146.939 101.854) (end 146.939 102.743) (width 0.25) (layer "F.Cu") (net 4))
 (segment (start 148.59 104.394) (end 154.432 104.394) (width 0.25) (layer "F.Cu") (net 4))
 (segment (start 146.939 102.743) (end 148.59 104.394) (width 0.25) (layer "F.Cu") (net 4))
 (via (at 146.939 101.854) (size 0.8) (drill 0.4) (layers "F.Cu" "B.Cu") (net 4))
 (segment (start 140.976 100.965) (end 140.897 101.044) (width 0.25) (layer "B.Cu") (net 4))
 (segment (start 146.939 101.854) (end 146.05 100.965) (width 0.25) (layer "B.Cu") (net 4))
 (segment (start 146.05 100.965) (end 140.976 100.965) (width 0.25) (layer "B.Cu") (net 4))
 (segment (start 143.764 100.965) (end 139.827 100.965) (width 0.25) (layer "F.Cu") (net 5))
 (segment (start 146.685 98.044) (end 143.764 100.965) (width 0.25) (layer "F.Cu") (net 5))
 (segment (start 151.56 98.044) (end 146.685 98.044) (width 0.25) (layer "F.Cu") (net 5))
 (via (at 139.827 100.965) (size 0.8) (drill 0.4) (layers "F.Cu" "B.Cu") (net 5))
 (segment (start 138.836 100.965) (end 138.757 101.044) (width 0.25) (layer "B.Cu") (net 5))
 (segment (start 139.827 100.965) (end 138.836 100.965) (width 0.25) (layer "B.Cu") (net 5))
 (segment (start 151.56 105.664) (end 145.823595 105.664) (width 0.25) (layer "F.Cu") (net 8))
 (segment (start 142.775595 102.616) (end 139.827 102.616) (width 0.25) (layer "F.Cu") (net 8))
 (segment (start 145.823595 105.664) (end 142.775595 102.616) (width 0.25) (layer "F.Cu") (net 8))
 (via (at 139.827 102.616) (size 0.8) (drill 0.4) (layers "F.Cu" "B.Cu") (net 8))
 (segment (start 138.785 102.616) (end 138.757 102.644) (width 0.25) (layer "B.Cu") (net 8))
 (segment (start 139.827 102.616) (end 138.785 102.616) (width 0.25) (layer "B.Cu") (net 8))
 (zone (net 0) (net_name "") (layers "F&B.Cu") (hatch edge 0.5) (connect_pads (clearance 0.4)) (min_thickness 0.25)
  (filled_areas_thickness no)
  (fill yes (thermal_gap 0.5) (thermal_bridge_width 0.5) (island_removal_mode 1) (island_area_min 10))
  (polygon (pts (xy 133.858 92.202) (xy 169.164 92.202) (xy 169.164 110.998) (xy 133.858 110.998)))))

